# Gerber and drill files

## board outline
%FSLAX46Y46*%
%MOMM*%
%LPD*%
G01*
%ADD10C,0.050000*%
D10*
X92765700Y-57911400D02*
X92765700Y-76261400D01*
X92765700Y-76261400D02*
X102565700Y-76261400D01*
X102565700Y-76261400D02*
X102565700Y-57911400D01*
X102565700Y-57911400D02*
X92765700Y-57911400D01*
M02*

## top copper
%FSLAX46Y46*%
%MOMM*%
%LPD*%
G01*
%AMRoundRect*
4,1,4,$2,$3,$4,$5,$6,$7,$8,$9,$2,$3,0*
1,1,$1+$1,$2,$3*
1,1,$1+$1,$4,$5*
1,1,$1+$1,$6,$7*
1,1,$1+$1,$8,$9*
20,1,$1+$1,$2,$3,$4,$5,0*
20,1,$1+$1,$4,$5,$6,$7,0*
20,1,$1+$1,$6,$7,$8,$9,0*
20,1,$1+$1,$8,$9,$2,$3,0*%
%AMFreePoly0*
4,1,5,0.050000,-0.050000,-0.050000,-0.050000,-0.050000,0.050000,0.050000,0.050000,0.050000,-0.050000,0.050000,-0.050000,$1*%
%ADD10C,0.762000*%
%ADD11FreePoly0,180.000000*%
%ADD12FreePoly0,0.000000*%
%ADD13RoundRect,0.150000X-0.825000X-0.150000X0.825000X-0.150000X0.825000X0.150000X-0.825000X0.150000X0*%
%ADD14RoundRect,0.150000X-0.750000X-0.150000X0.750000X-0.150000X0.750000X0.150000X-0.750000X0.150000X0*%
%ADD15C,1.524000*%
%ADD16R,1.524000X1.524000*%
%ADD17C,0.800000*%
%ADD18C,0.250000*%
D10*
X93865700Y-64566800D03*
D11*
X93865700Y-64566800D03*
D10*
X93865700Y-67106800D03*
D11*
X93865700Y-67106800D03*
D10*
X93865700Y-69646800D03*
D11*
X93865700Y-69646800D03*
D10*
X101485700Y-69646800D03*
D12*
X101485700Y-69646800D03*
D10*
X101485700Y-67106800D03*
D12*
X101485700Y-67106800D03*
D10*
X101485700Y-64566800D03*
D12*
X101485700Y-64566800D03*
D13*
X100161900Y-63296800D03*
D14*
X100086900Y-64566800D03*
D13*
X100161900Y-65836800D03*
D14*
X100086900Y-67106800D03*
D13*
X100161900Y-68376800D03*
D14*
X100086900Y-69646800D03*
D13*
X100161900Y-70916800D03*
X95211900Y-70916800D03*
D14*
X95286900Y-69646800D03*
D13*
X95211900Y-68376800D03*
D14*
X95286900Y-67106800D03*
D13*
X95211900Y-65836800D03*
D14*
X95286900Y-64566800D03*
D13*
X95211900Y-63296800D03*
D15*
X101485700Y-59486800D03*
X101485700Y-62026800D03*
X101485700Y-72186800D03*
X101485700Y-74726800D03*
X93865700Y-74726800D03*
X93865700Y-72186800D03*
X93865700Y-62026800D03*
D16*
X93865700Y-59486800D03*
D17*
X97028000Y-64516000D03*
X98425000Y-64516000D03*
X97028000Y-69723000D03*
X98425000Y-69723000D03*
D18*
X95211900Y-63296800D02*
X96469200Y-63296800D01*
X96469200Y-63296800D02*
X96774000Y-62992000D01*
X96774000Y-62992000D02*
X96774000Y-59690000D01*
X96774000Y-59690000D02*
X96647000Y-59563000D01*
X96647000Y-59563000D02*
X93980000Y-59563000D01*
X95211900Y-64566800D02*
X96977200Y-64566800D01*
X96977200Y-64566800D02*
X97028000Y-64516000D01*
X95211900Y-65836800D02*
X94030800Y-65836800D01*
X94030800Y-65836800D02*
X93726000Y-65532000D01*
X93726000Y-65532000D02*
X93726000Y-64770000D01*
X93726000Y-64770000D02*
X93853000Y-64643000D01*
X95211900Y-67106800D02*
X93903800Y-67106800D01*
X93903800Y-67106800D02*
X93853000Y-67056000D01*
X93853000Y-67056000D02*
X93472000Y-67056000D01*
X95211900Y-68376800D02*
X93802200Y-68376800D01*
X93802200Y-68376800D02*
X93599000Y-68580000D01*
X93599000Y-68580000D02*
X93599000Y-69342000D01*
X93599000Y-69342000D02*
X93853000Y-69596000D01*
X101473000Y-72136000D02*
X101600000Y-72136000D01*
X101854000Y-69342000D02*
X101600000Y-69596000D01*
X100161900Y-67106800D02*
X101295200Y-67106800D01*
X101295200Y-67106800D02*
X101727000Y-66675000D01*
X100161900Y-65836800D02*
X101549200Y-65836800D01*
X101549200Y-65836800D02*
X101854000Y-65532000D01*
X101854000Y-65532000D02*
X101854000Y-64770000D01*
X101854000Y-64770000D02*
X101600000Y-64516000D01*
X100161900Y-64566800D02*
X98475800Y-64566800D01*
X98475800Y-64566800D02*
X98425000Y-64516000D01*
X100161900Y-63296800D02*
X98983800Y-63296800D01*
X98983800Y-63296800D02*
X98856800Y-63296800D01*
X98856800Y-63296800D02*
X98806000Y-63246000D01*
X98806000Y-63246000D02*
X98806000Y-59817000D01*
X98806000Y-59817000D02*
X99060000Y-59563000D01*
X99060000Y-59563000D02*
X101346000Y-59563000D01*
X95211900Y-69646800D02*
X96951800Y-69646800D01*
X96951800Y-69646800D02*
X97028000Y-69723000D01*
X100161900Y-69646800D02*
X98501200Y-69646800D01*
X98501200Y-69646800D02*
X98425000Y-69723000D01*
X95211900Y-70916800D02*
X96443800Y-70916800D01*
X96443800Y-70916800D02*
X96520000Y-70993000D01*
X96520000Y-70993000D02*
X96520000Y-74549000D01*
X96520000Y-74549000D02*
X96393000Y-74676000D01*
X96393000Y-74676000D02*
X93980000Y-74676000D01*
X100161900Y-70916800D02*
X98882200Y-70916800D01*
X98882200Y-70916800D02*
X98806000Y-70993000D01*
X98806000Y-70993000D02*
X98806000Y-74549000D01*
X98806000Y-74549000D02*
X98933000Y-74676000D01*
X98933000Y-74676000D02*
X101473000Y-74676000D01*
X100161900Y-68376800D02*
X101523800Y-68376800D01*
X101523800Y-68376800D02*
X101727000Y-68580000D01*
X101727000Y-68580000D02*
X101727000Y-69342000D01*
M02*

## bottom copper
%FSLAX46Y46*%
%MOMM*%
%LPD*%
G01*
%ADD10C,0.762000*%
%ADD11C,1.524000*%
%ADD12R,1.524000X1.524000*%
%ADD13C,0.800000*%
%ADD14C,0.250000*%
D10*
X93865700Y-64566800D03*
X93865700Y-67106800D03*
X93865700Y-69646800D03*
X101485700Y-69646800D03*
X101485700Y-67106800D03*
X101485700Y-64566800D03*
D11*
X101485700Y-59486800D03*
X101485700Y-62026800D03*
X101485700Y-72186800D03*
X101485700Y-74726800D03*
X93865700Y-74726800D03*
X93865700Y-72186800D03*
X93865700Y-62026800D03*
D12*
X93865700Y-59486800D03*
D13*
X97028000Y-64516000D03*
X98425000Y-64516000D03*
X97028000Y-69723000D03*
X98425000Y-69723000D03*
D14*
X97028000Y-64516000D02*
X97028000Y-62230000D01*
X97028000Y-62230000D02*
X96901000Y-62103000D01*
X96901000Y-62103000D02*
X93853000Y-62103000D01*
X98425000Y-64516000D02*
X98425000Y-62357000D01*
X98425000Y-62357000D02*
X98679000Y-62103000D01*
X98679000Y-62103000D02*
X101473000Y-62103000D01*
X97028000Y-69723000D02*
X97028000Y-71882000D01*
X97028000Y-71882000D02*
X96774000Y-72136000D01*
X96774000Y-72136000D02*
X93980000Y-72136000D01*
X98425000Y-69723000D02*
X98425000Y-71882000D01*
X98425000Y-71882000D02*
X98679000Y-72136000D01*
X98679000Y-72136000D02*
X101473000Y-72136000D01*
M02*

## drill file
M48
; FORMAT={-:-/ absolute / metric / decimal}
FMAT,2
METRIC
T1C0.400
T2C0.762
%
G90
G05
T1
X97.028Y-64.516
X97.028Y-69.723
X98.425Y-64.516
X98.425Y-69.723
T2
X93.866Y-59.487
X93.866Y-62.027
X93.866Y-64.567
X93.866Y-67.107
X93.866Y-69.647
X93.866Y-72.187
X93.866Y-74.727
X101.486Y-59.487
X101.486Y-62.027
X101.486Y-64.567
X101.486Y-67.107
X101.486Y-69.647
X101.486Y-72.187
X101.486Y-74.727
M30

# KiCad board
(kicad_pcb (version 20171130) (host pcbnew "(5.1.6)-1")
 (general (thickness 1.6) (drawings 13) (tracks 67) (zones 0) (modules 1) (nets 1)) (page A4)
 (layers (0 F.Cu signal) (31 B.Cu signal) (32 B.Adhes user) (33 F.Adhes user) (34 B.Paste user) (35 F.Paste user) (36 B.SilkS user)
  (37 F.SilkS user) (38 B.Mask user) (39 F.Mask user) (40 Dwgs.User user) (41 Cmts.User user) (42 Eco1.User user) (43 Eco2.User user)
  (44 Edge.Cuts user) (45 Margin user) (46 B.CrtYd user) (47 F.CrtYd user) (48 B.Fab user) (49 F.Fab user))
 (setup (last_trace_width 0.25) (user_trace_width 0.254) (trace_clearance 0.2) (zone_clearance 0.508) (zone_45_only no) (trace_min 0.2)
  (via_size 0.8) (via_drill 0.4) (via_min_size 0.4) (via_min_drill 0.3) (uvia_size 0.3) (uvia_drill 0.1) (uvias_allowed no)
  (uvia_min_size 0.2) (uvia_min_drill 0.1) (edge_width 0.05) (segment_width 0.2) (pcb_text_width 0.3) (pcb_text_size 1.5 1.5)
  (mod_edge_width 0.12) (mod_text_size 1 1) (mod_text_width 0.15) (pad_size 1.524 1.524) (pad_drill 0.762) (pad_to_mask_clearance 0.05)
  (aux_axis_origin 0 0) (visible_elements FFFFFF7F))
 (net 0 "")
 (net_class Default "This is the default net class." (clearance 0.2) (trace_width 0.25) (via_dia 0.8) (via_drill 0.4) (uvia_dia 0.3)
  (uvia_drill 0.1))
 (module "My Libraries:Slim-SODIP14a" (layer F.Cu) (at 97.9297 67.1068)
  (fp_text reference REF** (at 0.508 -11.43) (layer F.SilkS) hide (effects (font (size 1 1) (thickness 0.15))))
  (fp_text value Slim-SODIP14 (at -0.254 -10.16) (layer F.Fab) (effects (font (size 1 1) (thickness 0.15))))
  (pad 3 thru_hole circle (at -4.064 -2.54 180) (size 0.762 0.762) (drill 0.762) (layers *.Cu B.Mask) (zone_connect 2))
  (pad 3 smd custom (at -4.064 -2.54 180) (size 0.1 0.1) (layers F.Cu F.Paste F.Mask) (zone_connect 2)
   (options (clearance outline) (anchor rect)) (primitives))
  (pad 4 thru_hole circle (at -4.064 0 180) (size 0.762 0.762) (drill 0.762) (layers *.Cu B.Mask) (zone_connect 2))
  (pad 4 smd custom (at -4.064 0 180) (size 0.1 0.1) (layers F.Cu F.Paste F.Mask) (zone_connect 2)
   (options (clearance outline) (anchor rect)) (primitives))
  (pad 5 thru_hole circle (at -4.064 2.54 180) (size 0.762 0.762) (drill 0.762) (layers *.Cu B.Mask) (zone_connect 2))
  (pad 5 smd custom (at -4.064 2.54 180) (size 0.1 0.1) (layers F.Cu F.Paste F.Mask) (zone_connect 2)
   (options (clearance outline) (anchor rect)) (primitives))
  (pad 10 thru_hole circle (at 3.556 2.54) (size 0.762 0.762) (drill 0.762) (layers *.Cu B.Mask) (zone_connect 2))
  (pad 10 smd custom (at 3.556 2.54) (size 0.1 0.1) (layers F.Cu F.Paste F.Mask) (zone_connect 2)
   (options (clearance outline) (anchor rect)) (primitives))
  (pad 11 thru_hole circle (at 3.556 0) (size 0.762 0.762) (drill 0.762) (layers *.Cu B.Mask) (zone_connect 2))
  (pad 11 smd custom (at 3.556 0) (size 0.1 0.1) (layers F.Cu F.Paste F.Mask) (zone_connect 2) (options (clearance outline) (anchor rect))
   (primitives))
  (pad 12 thru_hole circle (at 3.556 -2.54) (size 0.762 0.762) (drill 0.762) (layers *.Cu B.Mask) (zone_connect 2))
  (pad 12 smd custom (at 3.556 -2.54) (size 0.1 0.1) (layers F.Cu F.Paste F.Mask) (zone_connect 2)
   (options (clearance outline) (anchor rect)) (primitives))
  (pad 14 smd roundrect (at 2.2322 -3.81) (size 1.95 0.6) (layers F.Cu F.Paste F.Mask) (roundrect_rratio 0.25))
  (pad 13 smd roundrect (at 2.2322 -2.54) (size 1.8 0.6) (drill (offset -0.075 0)) (layers F.Cu F.Paste F.Mask) (roundrect_rratio 0.25))
  (pad 12 smd roundrect (at 2.2322 -1.27) (size 1.95 0.6) (layers F.Cu F.Paste F.Mask) (roundrect_rratio 0.25))
  (pad 11 smd roundrect (at 2.2322 0) (size 1.8 0.6) (drill (offset -0.075 0)) (layers F.Cu F.Paste F.Mask) (roundrect_rratio 0.25))
  (pad 10 smd roundrect (at 2.2322 1.27) (size 1.95 0.6) (layers F.Cu F.Paste F.Mask) (roundrect_rratio 0.25))
  (pad 9 smd roundrect (at 2.2322 2.54) (size 1.8 0.6) (drill (offset -0.075 0)) (layers F.Cu F.Paste F.Mask) (roundrect_rratio 0.25))
  (pad 8 smd roundrect (at 2.2322 3.81) (size 1.95 0.6) (layers F.Cu F.Paste F.Mask) (roundrect_rratio 0.25))
  (pad 7 smd roundrect (at -2.7178 3.81) (size 1.95 0.6) (layers F.Cu F.Paste F.Mask) (roundrect_rratio 0.25))
  (pad 6 smd roundrect (at -2.7178 2.54) (size 1.8 0.6) (drill (offset 0.075 0)) (layers F.Cu F.Paste F.Mask) (roundrect_rratio 0.25))
  (pad 5 smd roundrect (at -2.7178 1.27) (size 1.95 0.6) (layers F.Cu F.Paste F.Mask) (roundrect_rratio 0.25))
  (pad 4 smd roundrect (at -2.7178 0) (size 1.8 0.6) (drill (offset 0.075 0)) (layers F.Cu F.Paste F.Mask) (roundrect_rratio 0.25))
  (pad 3 smd roundrect (at -2.7178 -1.27) (size 1.95 0.6) (layers F.Cu F.Paste F.Mask) (roundrect_rratio 0.25))
  (pad 2 smd roundrect (at -2.7178 -2.54) (size 1.8 0.6) (drill (offset 0.075 0)) (layers F.Cu F.Paste F.Mask) (roundrect_rratio 0.25))
  (pad 1 smd roundrect (at -2.7178 -3.81) (size 1.95 0.6) (layers F.Cu F.Paste F.Mask) (roundrect_rratio 0.25))
  (pad 14 thru_hole circle (at 3.556 -7.62) (size 1.524 1.524) (drill 0.762) (layers *.Cu *.Mask))
  (pad 13 thru_hole circle (at 3.556 -5.08) (size 1.524 1.524) (drill 0.762) (layers *.Cu *.Mask))
  (pad 9 thru_hole circle (at 3.556 5.08) (size 1.524 1.524) (drill 0.762) (layers *.Cu *.Mask))
  (pad 8 thru_hole circle (at 3.556 7.62) (size 1.524 1.524) (drill 0.762) (layers *.Cu *.Mask))
  (pad 7 thru_hole circle (at -4.064 7.62) (size 1.524 1.524) (drill 0.762) (layers *.Cu *.Mask))
  (pad 6 thru_hole circle (at -4.064 5.08) (size 1.524 1.524) (drill 0.762) (layers *.Cu *.Mask))
  (pad 2 thru_hole circle (at -4.064 -5.08) (size 1.524 1.524) (drill 0.762) (layers *.Cu *.Mask))
  (pad 1 thru_hole rect (at -4.064 -7.62) (size 1.524 1.524) (drill 0.762) (layers *.Cu *.Mask)))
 (gr_line (start 92.7657 57.9114) (end 92.7657 76.2614) (layer Edge.Cuts) (width 0.05))
 (gr_line (start 92.7657 76.2614) (end 102.5657 76.2614) (layer Edge.Cuts) (width 0.05))
 (gr_line (start 102.5657 76.2614) (end 102.5657 57.9114) (layer Edge.Cuts) (width 0.05))
 (gr_line (start 102.5657 57.9114) (end 92.7657 57.9114) (layer Edge.Cuts) (width 0.05))
 (segment (start 95.2119 63.2968) (end 96.4692 63.2968) (width 0.25) (layer F.Cu) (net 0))
 (segment (start 96.4692 63.2968) (end 96.774 62.992) (width 0.25) (layer F.Cu) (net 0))
 (segment (start 96.774 62.992) (end 96.774 59.69) (width 0.25) (layer F.Cu) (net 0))
 (segment (start 96.774 59.69) (end 96.647 59.563) (width 0.25) (layer F.Cu) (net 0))
 (segment (start 96.647 59.563) (end 93.98 59.563) (width 0.25) (layer F.Cu) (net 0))
 (via (at 97.028 64.516) (size 0.8) (drill 0.4) (layers F.Cu B.Cu) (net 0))
 (segment (start 95.2119 64.5668) (end 96.9772 64.5668) (width 0.25) (layer F.Cu) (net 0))
 (segment (start 96.9772 64.5668) (end 97.028 64.516) (width 0.25) (layer F.Cu) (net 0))
 (segment (start 97.028 64.516) (end 97.028 62.23) (width 0.25) (layer B.Cu) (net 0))
 (segment (start 97.028 62.23) (end 96.901 62.103) (width 0.25) (layer B.Cu) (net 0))
 (segment (start 96.901 62.103) (end 93.853 62.103) (width 0.25) (layer B.Cu) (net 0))
 (segment (start 95.2119 65.8368) (end 94.0308 65.8368) (width 0.25) (layer F.Cu) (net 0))
 (segment (start 94.0308 65.8368) (end 93.726 65.532) (width 0.25) (layer F.Cu) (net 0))
 (segment (start 93.726 65.532) (end 93.726 64.77) (width 0.25) (layer F.Cu) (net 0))
 (segment (start 93.726 64.77) (end 93.853 64.643) (width 0.25) (layer F.Cu) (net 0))
 (segment (start 95.2119 67.1068) (end 93.9038 67.1068) (width 0.25) (layer F.Cu) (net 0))
 (segment (start 93.9038 67.1068) (end 93.853 67.056) (width 0.25) (layer F.Cu) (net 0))
 (segment (start 93.853 67.056) (end 93.472 67.056) (width 0.25) (layer F.Cu) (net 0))
 (segment (start 95.2119 68.3768) (end 93.8022 68.3768) (width 0.25) (layer F.Cu) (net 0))
 (segment (start 93.8022 68.3768) (end 93.599 68.58) (width 0.25) (layer F.Cu) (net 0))
 (segment (start 93.599 68.58) (end 93.599 69.342) (width 0.25) (layer F.Cu) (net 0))
 (segment (start 93.599 69.342) (end 93.853 69.596) (width 0.25) (layer F.Cu) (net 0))
 (segment (start 101.473 72.136) (end 101.6 72.136) (width 0.25) (layer F.Cu) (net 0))
 (segment (start 101.854 69.342) (end 101.6 69.596) (width 0.25) (layer F.Cu) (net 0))
 (segment (start 100.1619 67.1068) (end 101.2952 67.1068) (width 0.25) (layer F.Cu) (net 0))
 (segment (start 101.2952 67.1068) (end 101.727 66.675) (width 0.25) (layer F.Cu) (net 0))
 (segment (start 100.1619 65.8368) (end 101.5492 65.8368) (width 0.25) (layer F.Cu) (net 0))
 (segment (start 101.5492 65.8368) (end 101.854 65.532) (width 0.25) (layer F.Cu) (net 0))
 (segment (start 101.854 65.532) (end 101.854 64.77) (width 0.25) (layer F.Cu) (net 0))
 (segment (start 101.854 64.77) (end 101.6 64.516) (width 0.25) (layer F.Cu) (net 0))
 (via (at 98.425 64.516) (size 0.8) (drill 0.4) (layers F.Cu B.Cu) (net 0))
 (segment (start 100.1619 64.5668) (end 98.4758 64.5668) (width 0.25) (layer F.Cu) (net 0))
 (segment (start 98.4758 64.5668) (end 98.425 64.516) (width 0.25) (layer F.Cu) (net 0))
 (segment (start 98.425 64.516) (end 98.425 62.357) (width 0.25) (layer B.Cu) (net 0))
 (segment (start 98.425 62.357) (end 98.679 62.103) (width 0.25) (layer B.Cu) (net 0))
 (segment (start 98.679 62.103) (end 101.473 62.103) (width 0.25) (layer B.Cu) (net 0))
 (segment (start 100.1619 63.2968) (end 98.9838 63.2968) (width 0.25) (layer F.Cu) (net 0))
 (segment (start 98.9838 63.2968) (end 98.8568 63.2968) (width 0.25) (layer F.Cu) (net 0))
 (segment (start 98.8568 63.2968) (end 98.806 63.246) (width 0.25) (layer F.Cu) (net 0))
 (segment (start 98.806 63.246) (end 98.806 59.817) (width 0.25) (layer F.Cu) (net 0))
 (segment (start 98.806 59.817) (end 99.06 59.563) (width 0.25) (layer F.Cu) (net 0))
 (segment (start 99.06 59.563) (end 101.346 59.563) (width 0.25) (layer F.Cu) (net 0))
 (via (at 97.028 69.723) (size 0.8) (drill 0.4) (layers F.Cu B.Cu) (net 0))
 (segment (start 95.2119 69.6468) (end 96.9518 69.6468) (width 0.25) (layer F.Cu) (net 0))
 (segment (start 96.9518 69.6468) (end 97.028 69.723) (width 0.25) (layer F.Cu) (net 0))
 (segment (start 97.028 69.723) (end 97.028 71.882) (width 0.25) (layer B.Cu) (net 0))
 (segment (start 97.028 71.882) (end 96.774 72.136) (width 0.25) (layer B.Cu) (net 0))
 (segment (start 96.774 72.136) (end 93.98 72.136) (width 0.25) (layer B.Cu) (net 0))
 (via (at 98.425 69.723) (size 0.8) (drill 0.4) (layers F.Cu B.Cu) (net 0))
 (segment (start 100.1619 69.6468) (end 98.5012 69.6468) (width 0.25) (layer F.Cu) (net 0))
 (segment (start 98.5012 69.6468) (end 98.425 69.723) (width 0.25) (layer F.Cu) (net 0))
 (segment (start 98.425 69.723) (end 98.425 71.882) (width 0.25) (layer B.Cu) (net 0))
 (segment (start 98.425 71.882) (end 98.679 72.136) (width 0.25) (layer B.Cu) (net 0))
 (segment (start 98.679 72.136) (end 101.473 72.136) (width 0.25) (layer B.Cu) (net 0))
 (segment (start 95.2119 70.9168) (end 96.4438 70.9168) (width 0.25) (layer F.Cu) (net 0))
 (segment (start 96.4438 70.9168) (end 96.52 70.993) (width 0.25) (layer F.Cu) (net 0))
 (segment (start 96.52 70.993) (end 96.52 74.549) (width 0.25) (layer F.Cu) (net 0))
 (segment (start 96.52 74.549) (end 96.393 74.676) (width 0.25) (layer F.Cu) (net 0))
 (segment (start 96.393 74.676) (end 93.98 74.676) (width 0.25) (layer F.Cu) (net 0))
 (segment (start 100.1619 70.9168) (end 98.8822 70.9168) (width 0.25) (layer F.Cu) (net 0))
 (segment (start 98.8822 70.9168) (end 98.806 70.993) (width 0.25) (layer F.Cu) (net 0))
 (segment (start 98.806 70.993) (end 98.806 74.549) (width 0.25) (layer F.Cu) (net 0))
 (segment (start 98.806 74.549) (end 98.933 74.676) (width 0.25) (layer F.Cu) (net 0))
 (segment (start 98.933 74.676) (end 101.473 74.676) (width 0.25) (layer F.Cu) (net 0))
 (segment (start 100.1619 68.3768) (end 101.5238 68.3768) (width 0.25) (layer F.Cu) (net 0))
 (segment (start 101.5238 68.3768) (end 101.727 68.58) (width 0.25) (layer F.Cu) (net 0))
 (segment (start 101.727 68.58) (end 101.727 69.342) (width 0.25) (layer F.Cu) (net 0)))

